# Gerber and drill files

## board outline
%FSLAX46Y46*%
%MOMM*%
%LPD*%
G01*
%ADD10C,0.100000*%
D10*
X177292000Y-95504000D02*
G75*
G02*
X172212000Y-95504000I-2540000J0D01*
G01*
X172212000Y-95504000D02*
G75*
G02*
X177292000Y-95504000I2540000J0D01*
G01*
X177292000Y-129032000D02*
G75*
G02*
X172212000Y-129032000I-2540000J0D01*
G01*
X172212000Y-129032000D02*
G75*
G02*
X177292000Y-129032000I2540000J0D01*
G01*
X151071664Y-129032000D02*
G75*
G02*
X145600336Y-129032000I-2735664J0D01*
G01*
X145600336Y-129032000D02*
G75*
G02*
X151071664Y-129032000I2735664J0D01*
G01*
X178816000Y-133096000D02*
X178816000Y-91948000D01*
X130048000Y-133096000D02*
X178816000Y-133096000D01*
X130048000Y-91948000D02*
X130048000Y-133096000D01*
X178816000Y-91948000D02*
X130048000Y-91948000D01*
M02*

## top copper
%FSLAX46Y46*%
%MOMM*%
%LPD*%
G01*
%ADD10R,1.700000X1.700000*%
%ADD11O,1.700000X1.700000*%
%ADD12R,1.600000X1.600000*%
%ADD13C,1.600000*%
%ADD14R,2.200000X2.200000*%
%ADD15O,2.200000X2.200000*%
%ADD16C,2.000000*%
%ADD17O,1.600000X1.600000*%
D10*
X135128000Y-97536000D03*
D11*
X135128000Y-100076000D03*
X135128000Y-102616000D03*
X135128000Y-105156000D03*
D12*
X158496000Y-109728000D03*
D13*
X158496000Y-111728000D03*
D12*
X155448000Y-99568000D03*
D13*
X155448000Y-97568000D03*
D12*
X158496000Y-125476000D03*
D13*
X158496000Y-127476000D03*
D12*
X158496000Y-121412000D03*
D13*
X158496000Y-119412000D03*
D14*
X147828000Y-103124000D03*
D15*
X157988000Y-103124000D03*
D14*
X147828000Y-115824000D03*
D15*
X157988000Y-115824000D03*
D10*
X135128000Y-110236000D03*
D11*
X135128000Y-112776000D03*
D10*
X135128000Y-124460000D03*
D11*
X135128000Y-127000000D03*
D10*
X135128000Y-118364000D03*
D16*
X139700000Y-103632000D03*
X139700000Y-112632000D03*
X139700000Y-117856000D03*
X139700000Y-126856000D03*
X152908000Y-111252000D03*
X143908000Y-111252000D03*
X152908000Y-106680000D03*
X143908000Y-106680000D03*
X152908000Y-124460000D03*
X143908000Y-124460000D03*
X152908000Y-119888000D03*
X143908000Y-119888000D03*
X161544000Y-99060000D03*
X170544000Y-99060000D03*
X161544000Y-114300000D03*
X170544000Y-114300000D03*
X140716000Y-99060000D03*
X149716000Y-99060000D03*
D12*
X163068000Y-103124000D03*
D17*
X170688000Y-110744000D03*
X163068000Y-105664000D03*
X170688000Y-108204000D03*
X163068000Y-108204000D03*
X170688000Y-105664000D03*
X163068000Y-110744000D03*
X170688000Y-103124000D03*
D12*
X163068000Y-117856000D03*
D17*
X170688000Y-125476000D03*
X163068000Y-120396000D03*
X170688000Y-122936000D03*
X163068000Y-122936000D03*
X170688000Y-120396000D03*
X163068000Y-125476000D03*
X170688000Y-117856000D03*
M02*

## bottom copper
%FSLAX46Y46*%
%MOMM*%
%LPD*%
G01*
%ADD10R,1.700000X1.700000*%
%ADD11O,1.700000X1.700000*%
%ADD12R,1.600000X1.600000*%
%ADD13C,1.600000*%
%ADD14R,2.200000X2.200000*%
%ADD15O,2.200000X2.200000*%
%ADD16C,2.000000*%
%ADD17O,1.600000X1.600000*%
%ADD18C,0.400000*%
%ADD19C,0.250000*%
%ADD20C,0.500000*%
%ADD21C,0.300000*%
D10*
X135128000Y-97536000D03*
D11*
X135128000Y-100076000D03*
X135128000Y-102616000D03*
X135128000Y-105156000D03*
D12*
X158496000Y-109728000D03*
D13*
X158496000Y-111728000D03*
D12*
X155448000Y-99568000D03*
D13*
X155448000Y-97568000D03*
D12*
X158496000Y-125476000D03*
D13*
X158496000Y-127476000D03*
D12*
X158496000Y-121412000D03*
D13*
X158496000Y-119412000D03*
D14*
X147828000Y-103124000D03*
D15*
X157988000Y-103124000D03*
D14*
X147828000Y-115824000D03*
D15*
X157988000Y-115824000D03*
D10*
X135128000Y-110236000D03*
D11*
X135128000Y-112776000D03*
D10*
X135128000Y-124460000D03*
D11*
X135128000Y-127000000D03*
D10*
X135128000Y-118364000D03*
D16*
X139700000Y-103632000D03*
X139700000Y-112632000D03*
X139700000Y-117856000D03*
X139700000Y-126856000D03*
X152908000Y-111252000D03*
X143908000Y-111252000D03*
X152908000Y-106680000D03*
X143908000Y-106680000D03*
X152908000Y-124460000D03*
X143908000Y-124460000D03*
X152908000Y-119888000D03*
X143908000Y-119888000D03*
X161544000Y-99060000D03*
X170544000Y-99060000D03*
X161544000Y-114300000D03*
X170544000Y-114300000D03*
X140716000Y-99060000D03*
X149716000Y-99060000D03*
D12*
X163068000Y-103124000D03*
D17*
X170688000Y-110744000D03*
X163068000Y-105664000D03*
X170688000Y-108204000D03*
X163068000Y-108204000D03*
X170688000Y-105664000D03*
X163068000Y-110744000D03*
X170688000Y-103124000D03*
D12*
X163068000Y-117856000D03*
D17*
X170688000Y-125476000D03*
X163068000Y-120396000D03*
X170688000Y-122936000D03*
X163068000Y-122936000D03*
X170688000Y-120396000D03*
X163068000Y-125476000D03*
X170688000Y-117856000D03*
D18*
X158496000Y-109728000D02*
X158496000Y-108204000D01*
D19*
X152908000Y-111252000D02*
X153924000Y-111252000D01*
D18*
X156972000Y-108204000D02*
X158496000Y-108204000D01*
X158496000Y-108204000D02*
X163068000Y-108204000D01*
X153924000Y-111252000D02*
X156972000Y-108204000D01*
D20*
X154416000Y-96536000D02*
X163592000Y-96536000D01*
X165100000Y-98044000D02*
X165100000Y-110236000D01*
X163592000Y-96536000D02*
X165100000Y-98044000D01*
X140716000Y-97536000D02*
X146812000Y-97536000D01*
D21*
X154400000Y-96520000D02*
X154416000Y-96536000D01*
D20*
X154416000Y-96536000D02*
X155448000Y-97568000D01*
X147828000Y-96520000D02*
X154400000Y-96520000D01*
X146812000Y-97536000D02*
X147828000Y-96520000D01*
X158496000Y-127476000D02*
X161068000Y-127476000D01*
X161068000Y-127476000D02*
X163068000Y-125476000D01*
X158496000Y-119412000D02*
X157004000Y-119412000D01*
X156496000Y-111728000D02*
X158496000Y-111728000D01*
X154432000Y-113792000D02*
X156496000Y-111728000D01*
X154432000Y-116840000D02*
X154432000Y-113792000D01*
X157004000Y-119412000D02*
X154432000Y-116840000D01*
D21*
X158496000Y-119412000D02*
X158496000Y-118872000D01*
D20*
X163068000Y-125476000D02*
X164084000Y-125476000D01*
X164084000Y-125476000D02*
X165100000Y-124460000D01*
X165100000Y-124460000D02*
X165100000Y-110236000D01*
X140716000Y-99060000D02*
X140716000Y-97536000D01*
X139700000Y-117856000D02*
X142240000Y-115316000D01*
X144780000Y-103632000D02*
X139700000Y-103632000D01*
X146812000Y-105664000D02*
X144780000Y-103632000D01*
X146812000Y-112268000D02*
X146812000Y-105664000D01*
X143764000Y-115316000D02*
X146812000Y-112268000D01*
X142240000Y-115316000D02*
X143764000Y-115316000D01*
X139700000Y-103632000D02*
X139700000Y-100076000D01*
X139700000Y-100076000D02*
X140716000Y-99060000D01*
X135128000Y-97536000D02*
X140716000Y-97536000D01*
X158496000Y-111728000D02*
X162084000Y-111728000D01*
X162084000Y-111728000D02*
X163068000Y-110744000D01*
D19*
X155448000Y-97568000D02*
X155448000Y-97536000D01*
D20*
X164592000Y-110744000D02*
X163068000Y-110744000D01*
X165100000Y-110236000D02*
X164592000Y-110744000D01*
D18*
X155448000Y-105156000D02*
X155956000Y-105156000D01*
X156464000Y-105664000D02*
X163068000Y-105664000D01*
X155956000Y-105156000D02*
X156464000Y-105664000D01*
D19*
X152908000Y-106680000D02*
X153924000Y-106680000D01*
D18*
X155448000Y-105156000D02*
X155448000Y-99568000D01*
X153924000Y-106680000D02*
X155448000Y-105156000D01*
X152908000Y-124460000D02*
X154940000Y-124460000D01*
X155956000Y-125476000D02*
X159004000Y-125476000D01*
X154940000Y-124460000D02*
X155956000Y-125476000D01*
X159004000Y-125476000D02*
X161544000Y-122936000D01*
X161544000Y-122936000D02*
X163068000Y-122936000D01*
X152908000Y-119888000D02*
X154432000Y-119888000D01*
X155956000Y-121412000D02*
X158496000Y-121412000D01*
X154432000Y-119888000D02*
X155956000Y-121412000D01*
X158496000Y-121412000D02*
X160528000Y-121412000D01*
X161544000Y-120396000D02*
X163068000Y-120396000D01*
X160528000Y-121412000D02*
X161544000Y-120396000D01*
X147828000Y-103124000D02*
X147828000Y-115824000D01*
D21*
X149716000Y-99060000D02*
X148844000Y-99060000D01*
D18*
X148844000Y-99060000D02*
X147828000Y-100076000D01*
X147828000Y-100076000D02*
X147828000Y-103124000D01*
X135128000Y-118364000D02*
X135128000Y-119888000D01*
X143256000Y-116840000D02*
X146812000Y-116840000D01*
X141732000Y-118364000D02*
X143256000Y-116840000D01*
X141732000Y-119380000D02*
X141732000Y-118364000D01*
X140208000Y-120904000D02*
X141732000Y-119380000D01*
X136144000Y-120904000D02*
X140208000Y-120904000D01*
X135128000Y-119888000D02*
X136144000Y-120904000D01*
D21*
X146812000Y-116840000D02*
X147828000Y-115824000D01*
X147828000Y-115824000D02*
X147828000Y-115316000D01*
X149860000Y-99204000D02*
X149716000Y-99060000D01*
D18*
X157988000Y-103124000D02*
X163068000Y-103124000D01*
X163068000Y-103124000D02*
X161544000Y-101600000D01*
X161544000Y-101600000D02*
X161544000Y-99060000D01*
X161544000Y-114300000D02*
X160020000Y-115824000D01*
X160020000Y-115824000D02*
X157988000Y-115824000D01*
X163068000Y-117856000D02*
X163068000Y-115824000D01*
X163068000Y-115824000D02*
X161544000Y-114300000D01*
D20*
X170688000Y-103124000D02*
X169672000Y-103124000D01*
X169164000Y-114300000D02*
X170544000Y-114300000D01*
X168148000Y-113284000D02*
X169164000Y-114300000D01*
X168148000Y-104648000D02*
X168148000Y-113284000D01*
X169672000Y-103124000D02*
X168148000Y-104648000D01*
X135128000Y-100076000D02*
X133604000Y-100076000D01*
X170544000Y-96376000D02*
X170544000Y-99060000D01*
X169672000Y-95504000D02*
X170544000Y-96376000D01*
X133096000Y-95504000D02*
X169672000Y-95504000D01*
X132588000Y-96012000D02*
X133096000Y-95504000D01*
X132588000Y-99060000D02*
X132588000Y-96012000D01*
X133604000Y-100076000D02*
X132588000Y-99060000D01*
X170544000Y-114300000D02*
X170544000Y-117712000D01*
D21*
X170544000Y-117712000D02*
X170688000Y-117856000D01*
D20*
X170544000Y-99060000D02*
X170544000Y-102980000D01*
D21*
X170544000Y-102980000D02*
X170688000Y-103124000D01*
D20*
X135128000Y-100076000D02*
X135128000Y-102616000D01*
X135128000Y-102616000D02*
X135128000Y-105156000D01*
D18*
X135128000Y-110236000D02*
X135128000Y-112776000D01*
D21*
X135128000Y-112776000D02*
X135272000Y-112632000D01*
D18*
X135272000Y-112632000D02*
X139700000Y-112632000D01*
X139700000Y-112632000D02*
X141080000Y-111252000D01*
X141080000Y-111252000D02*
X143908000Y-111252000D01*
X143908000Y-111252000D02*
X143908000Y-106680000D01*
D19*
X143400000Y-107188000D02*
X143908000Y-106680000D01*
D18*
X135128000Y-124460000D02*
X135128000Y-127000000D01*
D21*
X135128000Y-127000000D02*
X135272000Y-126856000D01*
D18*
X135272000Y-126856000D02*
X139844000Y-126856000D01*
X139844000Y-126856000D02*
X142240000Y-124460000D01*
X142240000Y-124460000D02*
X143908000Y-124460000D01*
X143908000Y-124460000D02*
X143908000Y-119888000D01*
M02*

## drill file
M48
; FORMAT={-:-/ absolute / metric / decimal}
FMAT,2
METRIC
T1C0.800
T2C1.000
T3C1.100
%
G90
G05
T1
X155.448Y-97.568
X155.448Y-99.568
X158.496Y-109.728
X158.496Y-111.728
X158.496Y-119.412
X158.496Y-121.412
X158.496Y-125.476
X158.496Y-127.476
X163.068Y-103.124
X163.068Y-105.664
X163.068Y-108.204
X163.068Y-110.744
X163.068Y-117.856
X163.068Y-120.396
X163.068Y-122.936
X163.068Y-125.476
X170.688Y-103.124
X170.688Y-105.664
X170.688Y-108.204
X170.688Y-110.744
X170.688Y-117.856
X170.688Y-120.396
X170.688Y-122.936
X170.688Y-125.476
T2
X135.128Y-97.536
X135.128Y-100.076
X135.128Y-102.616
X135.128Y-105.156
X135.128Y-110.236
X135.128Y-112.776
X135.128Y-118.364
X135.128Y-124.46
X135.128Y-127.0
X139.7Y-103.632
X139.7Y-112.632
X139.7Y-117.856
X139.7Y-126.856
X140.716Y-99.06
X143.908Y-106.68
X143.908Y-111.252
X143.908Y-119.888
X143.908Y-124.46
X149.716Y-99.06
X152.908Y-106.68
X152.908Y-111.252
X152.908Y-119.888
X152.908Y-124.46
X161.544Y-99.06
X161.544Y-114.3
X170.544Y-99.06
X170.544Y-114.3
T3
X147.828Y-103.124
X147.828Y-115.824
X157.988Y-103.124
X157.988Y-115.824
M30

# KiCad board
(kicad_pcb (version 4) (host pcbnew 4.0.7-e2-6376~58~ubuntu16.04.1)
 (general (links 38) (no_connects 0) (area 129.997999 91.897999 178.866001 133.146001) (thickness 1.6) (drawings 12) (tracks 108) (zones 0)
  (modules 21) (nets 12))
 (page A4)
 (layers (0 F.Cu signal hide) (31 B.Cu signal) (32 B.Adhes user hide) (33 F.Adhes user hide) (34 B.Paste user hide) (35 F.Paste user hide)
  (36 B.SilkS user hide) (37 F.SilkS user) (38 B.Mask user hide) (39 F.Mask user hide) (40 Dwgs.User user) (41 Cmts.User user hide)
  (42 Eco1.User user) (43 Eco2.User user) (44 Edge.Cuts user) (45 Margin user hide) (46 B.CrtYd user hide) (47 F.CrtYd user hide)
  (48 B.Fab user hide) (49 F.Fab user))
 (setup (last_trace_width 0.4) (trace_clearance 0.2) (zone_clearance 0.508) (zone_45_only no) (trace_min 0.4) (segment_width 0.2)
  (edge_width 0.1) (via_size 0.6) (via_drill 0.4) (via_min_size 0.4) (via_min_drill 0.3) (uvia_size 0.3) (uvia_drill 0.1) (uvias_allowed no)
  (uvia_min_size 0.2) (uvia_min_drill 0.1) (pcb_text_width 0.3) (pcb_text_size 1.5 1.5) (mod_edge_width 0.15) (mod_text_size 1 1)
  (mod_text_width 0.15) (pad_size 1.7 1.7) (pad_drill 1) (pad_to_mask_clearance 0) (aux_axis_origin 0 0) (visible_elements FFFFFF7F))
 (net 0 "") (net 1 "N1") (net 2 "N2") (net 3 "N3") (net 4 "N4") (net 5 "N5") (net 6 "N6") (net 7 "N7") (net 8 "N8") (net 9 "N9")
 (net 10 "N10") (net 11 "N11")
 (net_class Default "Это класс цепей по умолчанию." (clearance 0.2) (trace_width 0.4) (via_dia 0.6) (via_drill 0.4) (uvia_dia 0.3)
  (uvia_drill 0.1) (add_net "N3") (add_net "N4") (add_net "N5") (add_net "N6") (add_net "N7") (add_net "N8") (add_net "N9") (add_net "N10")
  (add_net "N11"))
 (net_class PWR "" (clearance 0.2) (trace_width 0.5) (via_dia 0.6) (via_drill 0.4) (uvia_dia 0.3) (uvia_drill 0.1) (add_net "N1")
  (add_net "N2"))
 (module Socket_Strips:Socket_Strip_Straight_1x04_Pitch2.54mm (layer F.Cu) (at 135.128 97.536)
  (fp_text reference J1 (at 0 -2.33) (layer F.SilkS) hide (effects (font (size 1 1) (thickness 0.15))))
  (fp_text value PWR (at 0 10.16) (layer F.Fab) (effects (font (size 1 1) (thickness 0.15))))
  (pad 1 thru_hole rect (at 0 0) (size 1.7 1.7) (drill 1) (layers *.Cu *.Mask) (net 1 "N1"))
  (pad 2 thru_hole oval (at 0 2.54) (size 1.7 1.7) (drill 1) (layers *.Cu *.Mask) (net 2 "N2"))
  (pad 3 thru_hole oval (at 0 5.08) (size 1.7 1.7) (drill 1) (layers *.Cu B.Mask) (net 2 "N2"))
  (pad 4 thru_hole oval (at 0 7.62) (size 1.7 1.7) (drill 1) (layers *.Cu *.Mask) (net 2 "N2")))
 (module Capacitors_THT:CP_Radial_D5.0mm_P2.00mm (layer F.Cu) (at 158.496 109.728 270)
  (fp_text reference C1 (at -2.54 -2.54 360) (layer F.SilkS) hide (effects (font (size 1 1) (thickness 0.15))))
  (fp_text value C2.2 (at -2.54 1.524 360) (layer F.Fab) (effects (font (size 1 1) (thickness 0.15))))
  (pad 1 thru_hole rect (at 0 0 270) (size 1.6 1.6) (drill 0.8) (layers *.Cu *.Mask) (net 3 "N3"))
  (pad 2 thru_hole circle (at 2 0 270) (size 1.6 1.6) (drill 0.8) (layers *.Cu *.Mask) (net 1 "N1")))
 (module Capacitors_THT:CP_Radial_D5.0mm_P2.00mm (layer F.Cu) (at 155.448 99.568 90)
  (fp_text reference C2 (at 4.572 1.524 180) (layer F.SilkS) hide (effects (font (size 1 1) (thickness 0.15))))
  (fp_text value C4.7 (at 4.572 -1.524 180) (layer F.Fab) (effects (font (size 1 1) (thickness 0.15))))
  (pad 1 thru_hole rect (at 0 0 90) (size 1.6 1.6) (drill 0.8) (layers *.Cu *.Mask) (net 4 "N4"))
  (pad 2 thru_hole circle (at 2 0 90) (size 1.6 1.6) (drill 0.8) (layers *.Cu *.Mask) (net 1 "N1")))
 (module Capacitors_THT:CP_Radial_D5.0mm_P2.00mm (layer F.Cu) (at 158.496 125.476 270)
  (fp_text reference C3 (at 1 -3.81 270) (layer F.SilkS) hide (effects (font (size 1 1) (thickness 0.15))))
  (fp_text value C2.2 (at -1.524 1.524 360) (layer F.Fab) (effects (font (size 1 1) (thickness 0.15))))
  (pad 1 thru_hole rect (at 0 0 270) (size 1.6 1.6) (drill 0.8) (layers *.Cu *.Mask) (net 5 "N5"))
  (pad 2 thru_hole circle (at 2 0 270) (size 1.6 1.6) (drill 0.8) (layers *.Cu *.Mask) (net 1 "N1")))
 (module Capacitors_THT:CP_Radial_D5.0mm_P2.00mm (layer F.Cu) (at 158.496 121.412 90)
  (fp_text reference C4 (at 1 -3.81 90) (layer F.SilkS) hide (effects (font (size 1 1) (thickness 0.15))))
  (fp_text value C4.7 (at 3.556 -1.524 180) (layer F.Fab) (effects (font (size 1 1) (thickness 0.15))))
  (pad 1 thru_hole rect (at 0 0 90) (size 1.6 1.6) (drill 0.8) (layers *.Cu *.Mask) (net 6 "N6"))
  (pad 2 thru_hole circle (at 2 0 90) (size 1.6 1.6) (drill 0.8) (layers *.Cu *.Mask) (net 1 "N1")))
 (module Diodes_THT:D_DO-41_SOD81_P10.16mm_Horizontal (layer F.Cu) (at 147.828 103.124)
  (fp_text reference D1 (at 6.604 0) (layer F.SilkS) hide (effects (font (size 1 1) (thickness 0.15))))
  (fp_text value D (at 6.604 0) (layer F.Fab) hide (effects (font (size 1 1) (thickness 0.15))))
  (pad 1 thru_hole rect (at 0 0) (size 2.2 2.2) (drill 1.1) (layers *.Cu *.Mask) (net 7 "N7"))
  (pad 2 thru_hole oval (at 10.16 0) (size 2.2 2.2) (drill 1.1) (layers *.Cu *.Mask) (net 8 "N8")))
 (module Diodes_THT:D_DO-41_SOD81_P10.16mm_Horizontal (layer F.Cu) (at 147.828 115.824)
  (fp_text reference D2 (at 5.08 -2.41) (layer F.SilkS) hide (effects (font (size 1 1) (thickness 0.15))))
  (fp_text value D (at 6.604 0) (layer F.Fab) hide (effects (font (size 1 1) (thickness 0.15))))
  (pad 1 thru_hole rect (at 0 0) (size 2.2 2.2) (drill 1.1) (layers *.Cu *.Mask) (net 7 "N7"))
  (pad 2 thru_hole oval (at 10.16 0) (size 2.2 2.2) (drill 1.1) (layers *.Cu *.Mask) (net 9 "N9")))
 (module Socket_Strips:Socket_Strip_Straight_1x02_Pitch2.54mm (layer F.Cu) (at 135.128 110.236)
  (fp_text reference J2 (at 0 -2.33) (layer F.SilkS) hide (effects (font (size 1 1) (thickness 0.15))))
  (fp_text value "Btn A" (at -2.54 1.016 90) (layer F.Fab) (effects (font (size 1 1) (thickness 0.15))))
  (pad 1 thru_hole rect (at 0 0) (size 1.7 1.7) (drill 1) (layers *.Cu *.Mask) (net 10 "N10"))
  (pad 2 thru_hole oval (at 0 2.54) (size 1.7 1.7) (drill 1) (layers *.Cu *.Mask) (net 10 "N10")))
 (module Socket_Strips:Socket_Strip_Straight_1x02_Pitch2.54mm (layer F.Cu) (at 135.128 124.46)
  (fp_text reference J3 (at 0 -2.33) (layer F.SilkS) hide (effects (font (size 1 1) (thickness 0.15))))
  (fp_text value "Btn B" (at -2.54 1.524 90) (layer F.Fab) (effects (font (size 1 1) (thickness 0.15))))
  (pad 1 thru_hole rect (at 0 0) (size 1.7 1.7) (drill 1) (layers *.Cu *.Mask) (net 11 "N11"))
  (pad 2 thru_hole oval (at 0 2.54) (size 1.7 1.7) (drill 1) (layers *.Cu *.Mask) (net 11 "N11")))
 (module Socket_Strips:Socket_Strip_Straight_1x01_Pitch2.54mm (layer F.Cu) (at 135.128 118.364)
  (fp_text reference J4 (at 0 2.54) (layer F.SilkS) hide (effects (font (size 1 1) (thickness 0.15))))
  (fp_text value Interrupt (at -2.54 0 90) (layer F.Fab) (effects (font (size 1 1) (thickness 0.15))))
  (pad 1 thru_hole rect (at 0 0) (size 1.7 1.7) (drill 1) (layers *.Cu *.Mask) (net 7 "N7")))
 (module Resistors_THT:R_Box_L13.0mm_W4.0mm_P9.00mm (layer F.Cu) (at 139.7 103.632 270)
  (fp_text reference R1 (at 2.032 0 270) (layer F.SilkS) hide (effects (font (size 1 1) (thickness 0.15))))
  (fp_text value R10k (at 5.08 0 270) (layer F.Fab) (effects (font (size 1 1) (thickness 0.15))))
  (pad 1 thru_hole circle (at 0 0 270) (size 2 2) (drill 1) (layers *.Cu *.Mask) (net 1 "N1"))
  (pad 2 thru_hole circle (at 9 0 270) (size 2 2) (drill 1) (layers *.Cu *.Mask) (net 10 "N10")))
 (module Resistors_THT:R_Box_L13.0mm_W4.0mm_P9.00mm (layer F.Cu) (at 139.7 117.856 270)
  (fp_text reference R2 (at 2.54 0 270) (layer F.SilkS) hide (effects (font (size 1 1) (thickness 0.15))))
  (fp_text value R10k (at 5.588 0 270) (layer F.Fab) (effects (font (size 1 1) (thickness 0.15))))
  (pad 1 thru_hole circle (at 0 0 270) (size 2 2) (drill 1) (layers *.Cu *.Mask) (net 1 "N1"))
  (pad 2 thru_hole circle (at 9 0 270) (size 2 2) (drill 1) (layers *.Cu *.Mask) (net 11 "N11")))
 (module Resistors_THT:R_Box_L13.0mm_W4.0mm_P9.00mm (layer F.Cu) (at 152.908 111.252 180)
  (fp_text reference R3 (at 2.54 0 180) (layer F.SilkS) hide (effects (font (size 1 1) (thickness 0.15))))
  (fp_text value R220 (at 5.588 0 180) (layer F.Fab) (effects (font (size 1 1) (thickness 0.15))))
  (pad 1 thru_hole circle (at 0 0 180) (size 2 2) (drill 1) (layers *.Cu *.Mask) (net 3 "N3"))
  (pad 2 thru_hole circle (at 9 0 180) (size 2 2) (drill 1) (layers *.Cu *.Mask) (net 10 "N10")))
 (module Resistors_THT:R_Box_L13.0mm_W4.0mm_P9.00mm (layer F.Cu) (at 152.908 106.68 180)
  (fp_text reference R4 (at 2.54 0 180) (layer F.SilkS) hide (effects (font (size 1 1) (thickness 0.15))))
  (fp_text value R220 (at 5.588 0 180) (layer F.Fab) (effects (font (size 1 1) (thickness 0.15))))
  (pad 1 thru_hole circle (at 0 0 180) (size 2 2) (drill 1) (layers *.Cu *.Mask) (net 4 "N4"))
  (pad 2 thru_hole circle (at 9 0 180) (size 2 2) (drill 1) (layers *.Cu *.Mask) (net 10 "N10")))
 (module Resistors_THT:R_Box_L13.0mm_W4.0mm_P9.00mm (layer F.Cu) (at 152.908 124.46 180)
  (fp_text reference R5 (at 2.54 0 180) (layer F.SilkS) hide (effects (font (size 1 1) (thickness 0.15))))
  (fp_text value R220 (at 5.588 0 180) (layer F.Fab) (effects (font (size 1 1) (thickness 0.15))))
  (pad 1 thru_hole circle (at 0 0 180) (size 2 2) (drill 1) (layers *.Cu *.Mask) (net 5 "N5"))
  (pad 2 thru_hole circle (at 9 0 180) (size 2 2) (drill 1) (layers *.Cu *.Mask) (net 11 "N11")))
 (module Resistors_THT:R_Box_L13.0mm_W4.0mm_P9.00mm (layer F.Cu) (at 152.908 119.888 180)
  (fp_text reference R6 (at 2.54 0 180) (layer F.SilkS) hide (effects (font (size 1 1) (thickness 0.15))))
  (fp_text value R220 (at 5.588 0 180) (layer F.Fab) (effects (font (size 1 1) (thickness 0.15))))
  (pad 1 thru_hole circle (at 0 0 180) (size 2 2) (drill 1) (layers *.Cu *.Mask) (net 6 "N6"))
  (pad 2 thru_hole circle (at 9 0 180) (size 2 2) (drill 1) (layers *.Cu *.Mask) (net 11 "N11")))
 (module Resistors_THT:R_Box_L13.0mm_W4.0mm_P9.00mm (layer F.Cu) (at 161.544 99.06)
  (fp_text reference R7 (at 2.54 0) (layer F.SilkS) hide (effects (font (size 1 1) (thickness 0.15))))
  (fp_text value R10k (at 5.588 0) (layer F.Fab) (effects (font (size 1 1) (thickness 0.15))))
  (pad 1 thru_hole circle (at 0 0) (size 2 2) (drill 1) (layers *.Cu *.Mask) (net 8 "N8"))
  (pad 2 thru_hole circle (at 9 0) (size 2 2) (drill 1) (layers *.Cu *.Mask) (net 2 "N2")))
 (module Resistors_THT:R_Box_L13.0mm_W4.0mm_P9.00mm (layer F.Cu) (at 161.544 114.3)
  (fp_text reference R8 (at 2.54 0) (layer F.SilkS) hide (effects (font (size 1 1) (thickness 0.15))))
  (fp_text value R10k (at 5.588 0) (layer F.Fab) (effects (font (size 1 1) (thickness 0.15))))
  (pad 1 thru_hole circle (at 0 0) (size 2 2) (drill 1) (layers *.Cu *.Mask) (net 9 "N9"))
  (pad 2 thru_hole circle (at 9 0) (size 2 2) (drill 1) (layers *.Cu *.Mask) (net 2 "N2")))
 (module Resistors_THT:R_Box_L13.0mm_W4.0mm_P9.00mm (layer F.Cu) (at 140.716 99.06)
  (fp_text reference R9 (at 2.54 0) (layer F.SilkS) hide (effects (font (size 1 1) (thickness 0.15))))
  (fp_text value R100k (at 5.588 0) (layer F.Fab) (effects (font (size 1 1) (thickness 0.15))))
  (pad 1 thru_hole circle (at 0 0) (size 2 2) (drill 1) (layers *.Cu *.Mask) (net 1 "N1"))
  (pad 2 thru_hole circle (at 9 0) (size 2 2) (drill 1) (layers *.Cu *.Mask) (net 7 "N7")))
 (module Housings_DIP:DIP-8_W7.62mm (layer F.Cu) (at 163.068 103.124)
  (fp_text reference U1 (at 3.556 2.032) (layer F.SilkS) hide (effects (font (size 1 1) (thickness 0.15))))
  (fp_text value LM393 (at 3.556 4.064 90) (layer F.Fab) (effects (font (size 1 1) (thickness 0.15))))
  (pad 1 thru_hole rect (at 0 0) (size 1.6 1.6) (drill 0.8) (layers *.Cu *.Mask) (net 8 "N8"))
  (pad 5 thru_hole oval (at 7.62 7.62) (size 1.6 1.6) (drill 0.8) (layers *.Cu *.Mask))
  (pad 2 thru_hole oval (at 0 2.54) (size 1.6 1.6) (drill 0.8) (layers *.Cu *.Mask) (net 4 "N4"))
  (pad 6 thru_hole oval (at 7.62 5.08) (size 1.6 1.6) (drill 0.8) (layers *.Cu *.Mask))
  (pad 3 thru_hole oval (at 0 5.08) (size 1.6 1.6) (drill 0.8) (layers *.Cu *.Mask) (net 3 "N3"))
  (pad 7 thru_hole oval (at 7.62 2.54) (size 1.6 1.6) (drill 0.8) (layers *.Cu *.Mask))
  (pad 4 thru_hole oval (at 0 7.62) (size 1.6 1.6) (drill 0.8) (layers *.Cu *.Mask) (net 1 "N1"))
  (pad 8 thru_hole oval (at 7.62 0) (size 1.6 1.6) (drill 0.8) (layers *.Cu *.Mask) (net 2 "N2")))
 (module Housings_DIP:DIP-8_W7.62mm (layer F.Cu) (at 163.068 117.856)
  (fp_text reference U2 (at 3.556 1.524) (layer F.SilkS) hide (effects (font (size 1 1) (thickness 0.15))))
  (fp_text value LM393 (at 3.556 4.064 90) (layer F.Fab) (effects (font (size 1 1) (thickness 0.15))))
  (pad 1 thru_hole rect (at 0 0) (size 1.6 1.6) (drill 0.8) (layers *.Cu *.Mask) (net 9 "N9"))
  (pad 5 thru_hole oval (at 7.62 7.62) (size 1.6 1.6) (drill 0.8) (layers *.Cu *.Mask))
  (pad 2 thru_hole oval (at 0 2.54) (size 1.6 1.6) (drill 0.8) (layers *.Cu *.Mask) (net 6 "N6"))
  (pad 6 thru_hole oval (at 7.62 5.08) (size 1.6 1.6) (drill 0.8) (layers *.Cu *.Mask))
  (pad 3 thru_hole oval (at 0 5.08) (size 1.6 1.6) (drill 0.8) (layers *.Cu *.Mask) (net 5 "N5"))
  (pad 7 thru_hole oval (at 7.62 2.54) (size 1.6 1.6) (drill 0.8) (layers *.Cu *.Mask))
  (pad 4 thru_hole oval (at 0 7.62) (size 1.6 1.6) (drill 0.8) (layers *.Cu *.Mask) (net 1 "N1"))
  (pad 8 thru_hole oval (at 7.62 0) (size 1.6 1.6) (drill 0.8) (layers *.Cu *.Mask) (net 2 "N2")))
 (gr_circle (center 174.752 95.504) (end 177.292 95.504) (layer Edge.Cuts) (width 0.1))
 (gr_circle (center 174.752 129.032) (end 176.276 131.064) (layer Edge.Cuts) (width 0.1))
 (gr_circle (center 148.336 129.032) (end 150.876 130.048) (layer Edge.Cuts) (width 0.1))
 (gr_line (start 178.816 133.096) (end 178.816 91.948) (angle 90) (layer Edge.Cuts) (width 0.1))
 (gr_line (start 130.048 133.096) (end 178.816 133.096) (angle 90) (layer Edge.Cuts) (width 0.1))
 (gr_line (start 130.048 91.948) (end 130.048 133.096) (angle 90) (layer Edge.Cuts) (width 0.1))
 (gr_line (start 178.816 91.948) (end 130.048 91.948) (angle 90) (layer Edge.Cuts) (width 0.1))
 (segment (start 158.496 109.728) (end 158.496 108.204) (width 0.4) (layer B.Cu) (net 3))
 (segment (start 152.908 111.252) (end 153.924 111.252) (width 0.25) (layer B.Cu) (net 3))
 (segment (start 156.972 108.204) (end 158.496 108.204) (width 0.4) (layer B.Cu) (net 3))
 (segment (start 158.496 108.204) (end 163.068 108.204) (width 0.4) (layer B.Cu) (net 3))
 (segment (start 153.924 111.252) (end 156.972 108.204) (width 0.4) (layer B.Cu) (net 3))
 (segment (start 154.416 96.536) (end 163.592 96.536) (width 0.5) (layer B.Cu) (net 1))
 (segment (start 165.1 98.044) (end 165.1 110.236) (width 0.5) (layer B.Cu) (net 1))
 (segment (start 163.592 96.536) (end 165.1 98.044) (width 0.5) (layer B.Cu) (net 1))
 (segment (start 140.716 97.536) (end 146.812 97.536) (width 0.5) (layer B.Cu) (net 1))
 (segment (start 154.4 96.52) (end 154.416 96.536) (width 0.3) (layer B.Cu) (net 1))
 (segment (start 154.416 96.536) (end 155.448 97.568) (width 0.5) (layer B.Cu) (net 1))
 (segment (start 147.828 96.52) (end 154.4 96.52) (width 0.5) (layer B.Cu) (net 1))
 (segment (start 146.812 97.536) (end 147.828 96.52) (width 0.5) (layer B.Cu) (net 1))
 (segment (start 158.496 127.476) (end 161.068 127.476) (width 0.5) (layer B.Cu) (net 1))
 (segment (start 161.068 127.476) (end 163.068 125.476) (width 0.5) (layer B.Cu) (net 1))
 (segment (start 158.496 119.412) (end 157.004 119.412) (width 0.5) (layer B.Cu) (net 1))
 (segment (start 156.496 111.728) (end 158.496 111.728) (width 0.5) (layer B.Cu) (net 1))
 (segment (start 154.432 113.792) (end 156.496 111.728) (width 0.5) (layer B.Cu) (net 1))
 (segment (start 154.432 116.84) (end 154.432 113.792) (width 0.5) (layer B.Cu) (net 1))
 (segment (start 157.004 119.412) (end 154.432 116.84) (width 0.5) (layer B.Cu) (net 1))
 (segment (start 158.496 119.412) (end 158.496 118.872) (width 0.3) (layer B.Cu) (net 1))
 (segment (start 163.068 125.476) (end 164.084 125.476) (width 0.5) (layer B.Cu) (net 1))
 (segment (start 164.084 125.476) (end 165.1 124.46) (width 0.5) (layer B.Cu) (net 1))
 (segment (start 165.1 124.46) (end 165.1 110.236) (width 0.5) (layer B.Cu) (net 1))
 (segment (start 140.716 99.06) (end 140.716 97.536) (width 0.5) (layer B.Cu) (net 1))
 (segment (start 139.7 117.856) (end 142.24 115.316) (width 0.5) (layer B.Cu) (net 1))
 (segment (start 144.78 103.632) (end 139.7 103.632) (width 0.5) (layer B.Cu) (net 1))
 (segment (start 146.812 105.664) (end 144.78 103.632) (width 0.5) (layer B.Cu) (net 1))
 (segment (start 146.812 112.268) (end 146.812 105.664) (width 0.5) (layer B.Cu) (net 1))
 (segment (start 143.764 115.316) (end 146.812 112.268) (width 0.5) (layer B.Cu) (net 1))
 (segment (start 142.24 115.316) (end 143.764 115.316) (width 0.5) (layer B.Cu) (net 1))
 (segment (start 139.7 103.632) (end 139.7 100.076) (width 0.5) (layer B.Cu) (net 1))
 (segment (start 139.7 100.076) (end 140.716 99.06) (width 0.5) (layer B.Cu) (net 1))
 (segment (start 135.128 97.536) (end 140.716 97.536) (width 0.5) (layer B.Cu) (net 1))
 (segment (start 158.496 111.728) (end 162.084 111.728) (width 0.5) (layer B.Cu) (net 1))
 (segment (start 162.084 111.728) (end 163.068 110.744) (width 0.5) (layer B.Cu) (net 1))
 (segment (start 155.448 97.568) (end 155.448 97.536) (width 0.25) (layer B.Cu) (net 1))
 (segment (start 164.592 110.744) (end 163.068 110.744) (width 0.5) (layer B.Cu) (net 1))
 (segment (start 165.1 110.236) (end 164.592 110.744) (width 0.5) (layer B.Cu) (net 1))
 (segment (start 155.448 105.156) (end 155.956 105.156) (width 0.4) (layer B.Cu) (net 4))
 (segment (start 156.464 105.664) (end 163.068 105.664) (width 0.4) (layer B.Cu) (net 4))
 (segment (start 155.956 105.156) (end 156.464 105.664) (width 0.4) (layer B.Cu) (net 4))
 (segment (start 152.908 106.68) (end 153.924 106.68) (width 0.25) (layer B.Cu) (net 4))
 (segment (start 155.448 105.156) (end 155.448 99.568) (width 0.4) (layer B.Cu) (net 4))
 (segment (start 153.924 106.68) (end 155.448 105.156) (width 0.4) (layer B.Cu) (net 4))
 (segment (start 152.908 124.46) (end 154.94 124.46) (width 0.4) (layer B.Cu) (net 5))
 (segment (start 155.956 125.476) (end 159.004 125.476) (width 0.4) (layer B.Cu) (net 5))
 (segment (start 154.94 124.46) (end 155.956 125.476) (width 0.4) (layer B.Cu) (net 5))
 (segment (start 159.004 125.476) (end 161.544 122.936) (width 0.4) (layer B.Cu) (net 5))
 (segment (start 161.544 122.936) (end 163.068 122.936) (width 0.4) (layer B.Cu) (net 5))
 (segment (start 152.908 119.888) (end 154.432 119.888) (width 0.4) (layer B.Cu) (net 6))
 (segment (start 155.956 121.412) (end 158.496 121.412) (width 0.4) (layer B.Cu) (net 6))
 (segment (start 154.432 119.888) (end 155.956 121.412) (width 0.4) (layer B.Cu) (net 6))
 (segment (start 158.496 121.412) (end 160.528 121.412) (width 0.4) (layer B.Cu) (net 6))
 (segment (start 161.544 120.396) (end 163.068 120.396) (width 0.4) (layer B.Cu) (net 6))
 (segment (start 160.528 121.412) (end 161.544 120.396) (width 0.4) (layer B.Cu) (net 6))
 (segment (start 147.828 103.124) (end 147.828 115.824) (width 0.4) (layer B.Cu) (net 7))
 (segment (start 149.716 99.06) (end 148.844 99.06) (width 0.3) (layer B.Cu) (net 7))
 (segment (start 148.844 99.06) (end 147.828 100.076) (width 0.4) (layer B.Cu) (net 7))
 (segment (start 147.828 100.076) (end 147.828 103.124) (width 0.4) (layer B.Cu) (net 7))
 (segment (start 135.128 118.364) (end 135.128 119.888) (width 0.4) (layer B.Cu) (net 7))
 (segment (start 143.256 116.84) (end 146.812 116.84) (width 0.4) (layer B.Cu) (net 7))
 (segment (start 141.732 118.364) (end 143.256 116.84) (width 0.4) (layer B.Cu) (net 7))
 (segment (start 141.732 119.38) (end 141.732 118.364) (width 0.4) (layer B.Cu) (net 7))
 (segment (start 140.208 120.904) (end 141.732 119.38) (width 0.4) (layer B.Cu) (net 7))
 (segment (start 136.144 120.904) (end 140.208 120.904) (width 0.4) (layer B.Cu) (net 7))
 (segment (start 135.128 119.888) (end 136.144 120.904) (width 0.4) (layer B.Cu) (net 7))
 (segment (start 146.812 116.84) (end 147.828 115.824) (width 0.3) (layer B.Cu) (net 7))
 (segment (start 147.828 115.824) (end 147.828 115.316) (width 0.3) (layer B.Cu) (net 7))
 (segment (start 149.86 99.204) (end 149.716 99.06) (width 0.3) (layer B.Cu) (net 7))
 (segment (start 157.988 103.124) (end 163.068 103.124) (width 0.4) (layer B.Cu) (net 8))
 (segment (start 163.068 103.124) (end 161.544 101.6) (width 0.4) (layer B.Cu) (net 8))
 (segment (start 161.544 101.6) (end 161.544 99.06) (width 0.4) (layer B.Cu) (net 8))
 (segment (start 161.544 114.3) (end 160.02 115.824) (width 0.4) (layer B.Cu) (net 9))
 (segment (start 160.02 115.824) (end 157.988 115.824) (width 0.4) (layer B.Cu) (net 9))
 (segment (start 163.068 117.856) (end 163.068 115.824) (width 0.4) (layer B.Cu) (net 9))
 (segment (start 163.068 115.824) (end 161.544 114.3) (width 0.4) (layer B.Cu) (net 9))
 (segment (start 170.688 103.124) (end 169.672 103.124) (width 0.5) (layer B.Cu) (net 2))
 (segment (start 169.164 114.3) (end 170.544 114.3) (width 0.5) (layer B.Cu) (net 2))
 (segment (start 168.148 113.284) (end 169.164 114.3) (width 0.5) (layer B.Cu) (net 2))
 (segment (start 168.148 104.648) (end 168.148 113.284) (width 0.5) (layer B.Cu) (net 2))
 (segment (start 169.672 103.124) (end 168.148 104.648) (width 0.5) (layer B.Cu) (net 2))
 (segment (start 135.128 100.076) (end 133.604 100.076) (width 0.5) (layer B.Cu) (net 2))
 (segment (start 170.544 96.376) (end 170.544 99.06) (width 0.5) (layer B.Cu) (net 2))
 (segment (start 169.672 95.504) (end 170.544 96.376) (width 0.5) (layer B.Cu) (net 2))
 (segment (start 133.096 95.504) (end 169.672 95.504) (width 0.5) (layer B.Cu) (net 2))
 (segment (start 132.588 96.012) (end 133.096 95.504) (width 0.5) (layer B.Cu) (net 2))
 (segment (start 132.588 99.06) (end 132.588 96.012) (width 0.5) (layer B.Cu) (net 2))
 (segment (start 133.604 100.076) (end 132.588 99.06) (width 0.5) (layer B.Cu) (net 2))
 (segment (start 170.544 114.3) (end 170.544 117.712) (width 0.5) (layer B.Cu) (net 2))
 (segment (start 170.544 117.712) (end 170.688 117.856) (width 0.3) (layer B.Cu) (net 2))
 (segment (start 170.544 99.06) (end 170.544 102.98) (width 0.5) (layer B.Cu) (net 2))
 (segment (start 170.544 102.98) (end 170.688 103.124) (width 0.3) (layer B.Cu) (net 2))
 (segment (start 135.128 100.076) (end 135.128 102.616) (width 0.5) (layer B.Cu) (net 2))
 (segment (start 135.128 102.616) (end 135.128 105.156) (width 0.5) (layer B.Cu) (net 2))
 (segment (start 135.128 110.236) (end 135.128 112.776) (width 0.4) (layer B.Cu) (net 10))
 (segment (start 135.128 112.776) (end 135.272 112.632) (width 0.3) (layer B.Cu) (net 10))
 (segment (start 135.272 112.632) (end 139.7 112.632) (width 0.4) (layer B.Cu) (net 10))
 (segment (start 139.7 112.632) (end 141.08 111.252) (width 0.4) (layer B.Cu) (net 10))
 (segment (start 141.08 111.252) (end 143.908 111.252) (width 0.4) (layer B.Cu) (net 10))
 (segment (start 143.908 111.252) (end 143.908 106.68) (width 0.4) (layer B.Cu) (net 10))
 (segment (start 143.4 107.188) (end 143.908 106.68) (width 0.25) (layer B.Cu) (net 10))
 (segment (start 135.128 124.46) (end 135.128 127) (width 0.4) (layer B.Cu) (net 11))
 (segment (start 135.128 127) (end 135.272 126.856) (width 0.3) (layer B.Cu) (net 11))
 (segment (start 135.272 126.856) (end 139.844 126.856) (width 0.4) (layer B.Cu) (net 11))
 (segment (start 139.844 126.856) (end 142.24 124.46) (width 0.4) (layer B.Cu) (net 11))
 (segment (start 142.24 124.46) (end 143.908 124.46) (width 0.4) (layer B.Cu) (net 11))
 (segment (start 143.908 124.46) (end 143.908 119.888) (width 0.4) (layer B.Cu) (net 11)))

